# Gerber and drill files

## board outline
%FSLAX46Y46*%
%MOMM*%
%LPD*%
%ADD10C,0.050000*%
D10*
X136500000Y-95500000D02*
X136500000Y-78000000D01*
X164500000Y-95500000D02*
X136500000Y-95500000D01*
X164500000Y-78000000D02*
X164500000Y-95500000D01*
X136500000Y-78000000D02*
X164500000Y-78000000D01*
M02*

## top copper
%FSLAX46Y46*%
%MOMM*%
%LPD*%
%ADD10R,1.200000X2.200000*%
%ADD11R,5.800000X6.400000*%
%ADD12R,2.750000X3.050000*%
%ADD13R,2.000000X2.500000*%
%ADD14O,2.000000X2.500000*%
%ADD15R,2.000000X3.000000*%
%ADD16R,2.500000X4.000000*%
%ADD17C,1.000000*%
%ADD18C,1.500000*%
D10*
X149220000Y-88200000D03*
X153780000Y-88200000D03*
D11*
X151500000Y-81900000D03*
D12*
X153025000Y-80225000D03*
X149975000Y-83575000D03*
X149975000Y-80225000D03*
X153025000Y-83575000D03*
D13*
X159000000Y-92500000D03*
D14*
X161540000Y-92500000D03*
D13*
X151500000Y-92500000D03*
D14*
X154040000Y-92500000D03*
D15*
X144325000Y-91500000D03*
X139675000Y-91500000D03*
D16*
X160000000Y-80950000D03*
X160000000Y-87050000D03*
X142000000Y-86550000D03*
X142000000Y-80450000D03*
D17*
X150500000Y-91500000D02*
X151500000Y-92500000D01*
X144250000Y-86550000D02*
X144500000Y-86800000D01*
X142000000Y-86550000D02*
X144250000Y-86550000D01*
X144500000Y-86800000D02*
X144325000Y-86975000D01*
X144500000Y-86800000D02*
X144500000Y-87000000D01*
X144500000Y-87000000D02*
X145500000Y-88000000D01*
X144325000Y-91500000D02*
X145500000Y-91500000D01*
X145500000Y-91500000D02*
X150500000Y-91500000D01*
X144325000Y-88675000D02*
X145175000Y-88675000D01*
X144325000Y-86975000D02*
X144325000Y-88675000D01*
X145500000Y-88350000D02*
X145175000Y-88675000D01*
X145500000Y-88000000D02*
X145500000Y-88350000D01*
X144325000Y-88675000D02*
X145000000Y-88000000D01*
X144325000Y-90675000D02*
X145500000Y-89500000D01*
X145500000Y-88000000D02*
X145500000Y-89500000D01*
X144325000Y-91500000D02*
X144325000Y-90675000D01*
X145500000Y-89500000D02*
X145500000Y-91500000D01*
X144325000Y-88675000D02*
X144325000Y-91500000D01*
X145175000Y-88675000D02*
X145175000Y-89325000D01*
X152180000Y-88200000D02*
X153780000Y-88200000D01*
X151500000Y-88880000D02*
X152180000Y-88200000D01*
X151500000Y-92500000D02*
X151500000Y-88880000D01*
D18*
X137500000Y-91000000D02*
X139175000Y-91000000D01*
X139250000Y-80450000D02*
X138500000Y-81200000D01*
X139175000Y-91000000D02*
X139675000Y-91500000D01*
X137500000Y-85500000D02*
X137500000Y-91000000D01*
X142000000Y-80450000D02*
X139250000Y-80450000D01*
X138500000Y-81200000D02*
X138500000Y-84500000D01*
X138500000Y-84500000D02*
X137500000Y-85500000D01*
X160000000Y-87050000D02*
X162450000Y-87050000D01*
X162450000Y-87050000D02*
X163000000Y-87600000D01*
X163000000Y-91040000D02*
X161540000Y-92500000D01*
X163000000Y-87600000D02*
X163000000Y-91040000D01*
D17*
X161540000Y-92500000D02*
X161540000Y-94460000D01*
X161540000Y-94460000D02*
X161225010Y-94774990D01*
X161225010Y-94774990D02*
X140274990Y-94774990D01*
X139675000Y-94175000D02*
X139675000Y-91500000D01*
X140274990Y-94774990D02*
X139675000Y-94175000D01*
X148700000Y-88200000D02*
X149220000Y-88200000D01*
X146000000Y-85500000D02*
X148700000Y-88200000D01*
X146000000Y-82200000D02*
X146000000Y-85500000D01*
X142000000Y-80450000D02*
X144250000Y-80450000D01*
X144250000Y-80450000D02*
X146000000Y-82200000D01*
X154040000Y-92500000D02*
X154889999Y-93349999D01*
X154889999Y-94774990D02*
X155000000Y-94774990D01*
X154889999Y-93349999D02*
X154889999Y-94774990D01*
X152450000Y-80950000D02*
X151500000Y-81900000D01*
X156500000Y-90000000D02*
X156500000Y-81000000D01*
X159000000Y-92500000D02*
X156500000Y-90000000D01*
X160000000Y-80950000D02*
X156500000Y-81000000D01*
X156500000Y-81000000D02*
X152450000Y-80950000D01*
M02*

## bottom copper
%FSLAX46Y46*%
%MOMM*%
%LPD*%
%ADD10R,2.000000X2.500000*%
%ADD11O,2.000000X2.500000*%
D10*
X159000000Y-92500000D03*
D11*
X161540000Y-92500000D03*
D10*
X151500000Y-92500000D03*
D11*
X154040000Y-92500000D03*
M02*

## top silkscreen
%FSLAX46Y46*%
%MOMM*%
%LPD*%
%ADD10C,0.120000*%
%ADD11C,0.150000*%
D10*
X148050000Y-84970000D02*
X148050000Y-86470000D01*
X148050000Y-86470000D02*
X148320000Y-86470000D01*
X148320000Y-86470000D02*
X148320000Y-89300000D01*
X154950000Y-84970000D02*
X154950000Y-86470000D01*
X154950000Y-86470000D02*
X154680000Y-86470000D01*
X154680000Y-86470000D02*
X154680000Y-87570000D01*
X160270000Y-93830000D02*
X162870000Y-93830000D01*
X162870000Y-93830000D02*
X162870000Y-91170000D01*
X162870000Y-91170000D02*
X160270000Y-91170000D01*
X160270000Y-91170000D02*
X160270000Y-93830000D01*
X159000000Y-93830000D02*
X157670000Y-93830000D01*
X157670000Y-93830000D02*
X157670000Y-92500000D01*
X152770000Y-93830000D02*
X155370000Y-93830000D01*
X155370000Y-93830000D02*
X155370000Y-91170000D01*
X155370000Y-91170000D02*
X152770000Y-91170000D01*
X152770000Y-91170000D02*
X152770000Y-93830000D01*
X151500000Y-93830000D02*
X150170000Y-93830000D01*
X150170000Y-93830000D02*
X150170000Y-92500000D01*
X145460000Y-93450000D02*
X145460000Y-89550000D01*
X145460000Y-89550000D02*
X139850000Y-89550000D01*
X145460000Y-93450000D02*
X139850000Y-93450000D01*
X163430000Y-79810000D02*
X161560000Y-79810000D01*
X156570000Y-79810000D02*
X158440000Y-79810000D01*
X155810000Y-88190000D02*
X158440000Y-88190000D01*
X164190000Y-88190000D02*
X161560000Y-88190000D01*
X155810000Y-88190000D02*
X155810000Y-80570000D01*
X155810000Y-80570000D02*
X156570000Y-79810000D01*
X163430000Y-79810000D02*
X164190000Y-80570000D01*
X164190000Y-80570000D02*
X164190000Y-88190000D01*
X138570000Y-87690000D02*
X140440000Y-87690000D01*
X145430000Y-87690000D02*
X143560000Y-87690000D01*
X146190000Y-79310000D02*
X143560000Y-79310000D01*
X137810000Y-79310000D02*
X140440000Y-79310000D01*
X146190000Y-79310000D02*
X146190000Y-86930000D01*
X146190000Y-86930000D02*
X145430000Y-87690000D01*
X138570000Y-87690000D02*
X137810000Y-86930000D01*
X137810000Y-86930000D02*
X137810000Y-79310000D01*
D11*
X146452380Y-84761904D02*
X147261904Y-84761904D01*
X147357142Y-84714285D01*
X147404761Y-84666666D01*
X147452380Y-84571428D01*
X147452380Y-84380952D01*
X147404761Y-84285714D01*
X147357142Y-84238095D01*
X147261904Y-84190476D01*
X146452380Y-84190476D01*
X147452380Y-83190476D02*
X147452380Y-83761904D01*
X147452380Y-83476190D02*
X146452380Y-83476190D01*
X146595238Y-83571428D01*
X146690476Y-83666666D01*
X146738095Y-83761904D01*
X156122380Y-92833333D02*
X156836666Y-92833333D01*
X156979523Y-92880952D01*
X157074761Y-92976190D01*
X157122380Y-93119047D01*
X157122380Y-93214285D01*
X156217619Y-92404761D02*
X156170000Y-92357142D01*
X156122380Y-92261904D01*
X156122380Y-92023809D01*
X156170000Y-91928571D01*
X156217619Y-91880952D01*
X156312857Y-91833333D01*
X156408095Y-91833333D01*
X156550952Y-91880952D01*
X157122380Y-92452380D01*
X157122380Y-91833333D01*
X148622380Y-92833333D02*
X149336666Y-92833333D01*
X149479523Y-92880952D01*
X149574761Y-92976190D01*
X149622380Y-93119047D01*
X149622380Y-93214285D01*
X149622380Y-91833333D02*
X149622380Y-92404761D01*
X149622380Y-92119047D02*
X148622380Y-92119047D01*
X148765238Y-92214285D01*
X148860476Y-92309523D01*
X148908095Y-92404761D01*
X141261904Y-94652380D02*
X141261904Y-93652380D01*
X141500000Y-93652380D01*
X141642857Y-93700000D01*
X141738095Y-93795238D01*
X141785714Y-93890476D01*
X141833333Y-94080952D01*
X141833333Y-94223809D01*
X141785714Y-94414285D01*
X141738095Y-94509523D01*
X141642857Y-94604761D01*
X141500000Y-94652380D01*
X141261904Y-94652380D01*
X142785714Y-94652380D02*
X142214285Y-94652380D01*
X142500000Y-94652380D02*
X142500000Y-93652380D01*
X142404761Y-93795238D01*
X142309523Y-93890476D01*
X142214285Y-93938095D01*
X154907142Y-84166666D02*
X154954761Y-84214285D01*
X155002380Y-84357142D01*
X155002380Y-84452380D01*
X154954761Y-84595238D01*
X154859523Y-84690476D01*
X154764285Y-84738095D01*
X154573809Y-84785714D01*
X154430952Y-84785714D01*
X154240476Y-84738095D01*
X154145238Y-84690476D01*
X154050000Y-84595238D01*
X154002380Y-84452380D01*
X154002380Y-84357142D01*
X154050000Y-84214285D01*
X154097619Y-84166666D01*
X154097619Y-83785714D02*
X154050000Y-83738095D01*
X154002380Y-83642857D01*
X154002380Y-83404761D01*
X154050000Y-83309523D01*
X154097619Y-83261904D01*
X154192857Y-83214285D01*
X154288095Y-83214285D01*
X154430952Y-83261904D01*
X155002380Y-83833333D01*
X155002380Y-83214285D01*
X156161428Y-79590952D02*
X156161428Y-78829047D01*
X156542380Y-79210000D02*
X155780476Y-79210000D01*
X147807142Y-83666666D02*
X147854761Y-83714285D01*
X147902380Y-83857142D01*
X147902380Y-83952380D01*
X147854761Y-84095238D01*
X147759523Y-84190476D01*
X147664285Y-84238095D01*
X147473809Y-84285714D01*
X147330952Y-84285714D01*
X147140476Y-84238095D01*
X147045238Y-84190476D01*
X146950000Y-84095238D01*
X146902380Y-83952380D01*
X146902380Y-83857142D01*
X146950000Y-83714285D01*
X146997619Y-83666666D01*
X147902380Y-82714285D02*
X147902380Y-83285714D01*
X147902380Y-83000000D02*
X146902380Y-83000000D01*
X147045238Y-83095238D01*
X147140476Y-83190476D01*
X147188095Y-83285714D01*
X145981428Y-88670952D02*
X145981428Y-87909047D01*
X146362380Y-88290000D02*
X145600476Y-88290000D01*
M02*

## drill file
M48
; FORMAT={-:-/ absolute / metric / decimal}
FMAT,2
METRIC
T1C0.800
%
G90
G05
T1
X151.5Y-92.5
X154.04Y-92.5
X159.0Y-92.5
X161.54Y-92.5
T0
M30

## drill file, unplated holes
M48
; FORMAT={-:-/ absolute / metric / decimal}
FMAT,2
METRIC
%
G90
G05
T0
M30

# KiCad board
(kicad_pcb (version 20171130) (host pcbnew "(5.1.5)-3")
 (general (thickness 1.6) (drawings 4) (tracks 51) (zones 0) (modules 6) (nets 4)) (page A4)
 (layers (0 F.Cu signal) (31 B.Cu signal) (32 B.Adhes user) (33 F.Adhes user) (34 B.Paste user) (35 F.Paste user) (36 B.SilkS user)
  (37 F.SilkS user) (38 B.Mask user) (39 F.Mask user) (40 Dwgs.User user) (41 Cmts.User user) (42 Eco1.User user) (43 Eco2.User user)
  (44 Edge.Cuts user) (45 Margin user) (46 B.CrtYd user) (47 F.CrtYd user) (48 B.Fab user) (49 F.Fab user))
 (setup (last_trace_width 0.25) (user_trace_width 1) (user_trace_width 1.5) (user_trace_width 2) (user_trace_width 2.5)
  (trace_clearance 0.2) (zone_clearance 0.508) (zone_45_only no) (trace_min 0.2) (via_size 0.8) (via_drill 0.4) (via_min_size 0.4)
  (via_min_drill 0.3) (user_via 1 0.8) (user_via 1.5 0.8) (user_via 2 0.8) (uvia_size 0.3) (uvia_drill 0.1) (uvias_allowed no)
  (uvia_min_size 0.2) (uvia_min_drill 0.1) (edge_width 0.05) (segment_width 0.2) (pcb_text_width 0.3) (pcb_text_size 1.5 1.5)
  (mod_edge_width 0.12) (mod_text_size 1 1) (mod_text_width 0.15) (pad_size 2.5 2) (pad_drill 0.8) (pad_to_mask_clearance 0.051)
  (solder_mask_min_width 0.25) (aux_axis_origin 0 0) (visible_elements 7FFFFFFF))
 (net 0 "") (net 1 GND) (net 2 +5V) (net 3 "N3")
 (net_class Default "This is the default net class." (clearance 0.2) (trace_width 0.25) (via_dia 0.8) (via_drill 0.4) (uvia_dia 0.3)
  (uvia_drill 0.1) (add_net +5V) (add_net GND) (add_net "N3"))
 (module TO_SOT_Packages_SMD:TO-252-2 (layer F.Cu) (at 151.5 84 90)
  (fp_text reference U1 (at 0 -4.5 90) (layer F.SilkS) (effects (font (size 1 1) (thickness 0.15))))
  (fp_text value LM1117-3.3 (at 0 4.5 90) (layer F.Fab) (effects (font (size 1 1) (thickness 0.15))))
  (fp_line (start -0.97 -3.45) (end -2.47 -3.45) (layer F.SilkS) (width 0.12))
  (fp_line (start -2.47 -3.45) (end -2.47 -3.18) (layer F.SilkS) (width 0.12))
  (fp_line (start -2.47 -3.18) (end -5.3 -3.18) (layer F.SilkS) (width 0.12))
  (fp_line (start -0.97 3.45) (end -2.47 3.45) (layer F.SilkS) (width 0.12))
  (fp_line (start -2.47 3.45) (end -2.47 3.18) (layer F.SilkS) (width 0.12))
  (fp_line (start -2.47 3.18) (end -3.57 3.18) (layer F.SilkS) (width 0.12))
  (pad 1 smd rect (at -4.2 -2.28 90) (size 2.2 1.2) (layers F.Cu F.Paste F.Mask) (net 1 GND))
  (pad 3 smd rect (at -4.2 2.28 90) (size 2.2 1.2) (layers F.Cu F.Paste F.Mask) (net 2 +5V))
  (pad 2 smd rect (at 2.1 0 90) (size 6.4 5.8) (layers F.Cu F.Mask) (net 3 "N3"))
  (pad 2 smd rect (at 3.775 1.525 90) (size 3.05 2.75) (layers F.Cu F.Paste) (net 3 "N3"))
  (pad 2 smd rect (at 0.425 -1.525 90) (size 3.05 2.75) (layers F.Cu F.Paste) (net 3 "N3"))
  (pad 2 smd rect (at 3.775 -1.525 90) (size 3.05 2.75) (layers F.Cu F.Paste) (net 3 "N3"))
  (pad 2 smd rect (at 0.425 1.525 90) (size 3.05 2.75) (layers F.Cu F.Paste) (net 3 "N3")))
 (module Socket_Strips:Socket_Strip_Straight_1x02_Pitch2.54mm (layer F.Cu) (at 159 92.5 90)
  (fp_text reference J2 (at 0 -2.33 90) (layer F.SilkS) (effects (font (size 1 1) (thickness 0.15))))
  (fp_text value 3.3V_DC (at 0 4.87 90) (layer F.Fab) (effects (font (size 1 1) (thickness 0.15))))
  (fp_line (start -1.33 1.27) (end -1.33 3.87) (layer F.SilkS) (width 0.12))
  (fp_line (start -1.33 3.87) (end 1.33 3.87) (layer F.SilkS) (width 0.12))
  (fp_line (start 1.33 3.87) (end 1.33 1.27) (layer F.SilkS) (width 0.12))
  (fp_line (start 1.33 1.27) (end -1.33 1.27) (layer F.SilkS) (width 0.12))
  (fp_line (start -1.33 0) (end -1.33 -1.33) (layer F.SilkS) (width 0.12))
  (fp_line (start -1.33 -1.33) (end 0 -1.33) (layer F.SilkS) (width 0.12))
  (pad 1 thru_hole rect (at 0 0 90) (size 2.5 2) (drill 0.8) (layers *.Cu *.Mask) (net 3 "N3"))
  (pad 2 thru_hole oval (at 0 2.54 90) (size 2.5 2) (drill 0.8) (layers *.Cu *.Mask) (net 1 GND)))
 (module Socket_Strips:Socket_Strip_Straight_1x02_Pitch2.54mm (layer F.Cu) (at 151.5 92.5 90)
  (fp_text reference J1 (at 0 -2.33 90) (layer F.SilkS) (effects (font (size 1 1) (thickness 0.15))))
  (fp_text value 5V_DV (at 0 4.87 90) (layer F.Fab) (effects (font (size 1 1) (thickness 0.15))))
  (fp_line (start -1.33 1.27) (end -1.33 3.87) (layer F.SilkS) (width 0.12))
  (fp_line (start -1.33 3.87) (end 1.33 3.87) (layer F.SilkS) (width 0.12))
  (fp_line (start 1.33 3.87) (end 1.33 1.27) (layer F.SilkS) (width 0.12))
  (fp_line (start 1.33 1.27) (end -1.33 1.27) (layer F.SilkS) (width 0.12))
  (fp_line (start -1.33 0) (end -1.33 -1.33) (layer F.SilkS) (width 0.12))
  (fp_line (start -1.33 -1.33) (end 0 -1.33) (layer F.SilkS) (width 0.12))
  (pad 1 thru_hole rect (at 0 0 90) (size 2.5 2) (drill 0.8) (layers *.Cu *.Mask) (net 2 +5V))
  (pad 2 thru_hole oval (at 0 2.54 90) (size 2.5 2) (drill 0.8) (layers *.Cu *.Mask) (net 1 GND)))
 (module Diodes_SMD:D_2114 (layer F.Cu) (at 142 91.5 180)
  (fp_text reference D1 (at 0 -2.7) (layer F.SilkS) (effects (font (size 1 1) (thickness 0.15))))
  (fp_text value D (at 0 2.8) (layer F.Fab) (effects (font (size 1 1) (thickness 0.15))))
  (fp_line (start -3.46 -1.95) (end -3.46 1.95) (layer F.SilkS) (width 0.12))
  (fp_line (start -3.46 1.95) (end 2.15 1.95) (layer F.SilkS) (width 0.12))
  (fp_line (start -3.46 -1.95) (end 2.15 -1.95) (layer F.SilkS) (width 0.12))
  (pad 1 smd rect (at -2.325 0 180) (size 2 3) (layers F.Cu F.Paste F.Mask) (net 2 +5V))
  (pad 2 smd rect (at 2.325 0 180) (size 2 3) (layers F.Cu F.Paste F.Mask) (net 1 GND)))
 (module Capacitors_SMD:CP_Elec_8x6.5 (layer F.Cu) (at 160 84 270)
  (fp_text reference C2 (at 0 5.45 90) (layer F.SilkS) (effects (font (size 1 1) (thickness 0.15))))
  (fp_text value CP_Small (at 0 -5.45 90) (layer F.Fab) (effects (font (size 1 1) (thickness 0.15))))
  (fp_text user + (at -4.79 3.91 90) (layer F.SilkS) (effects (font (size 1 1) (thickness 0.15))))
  (fp_line (start -4.19 -3.43) (end -4.19 -1.56) (layer F.SilkS) (width 0.12))
  (fp_line (start -4.19 3.43) (end -4.19 1.56) (layer F.SilkS) (width 0.12))
  (fp_line (start 4.19 4.19) (end 4.19 1.56) (layer F.SilkS) (width 0.12))
  (fp_line (start 4.19 -4.19) (end 4.19 -1.56) (layer F.SilkS) (width 0.12))
  (fp_line (start 4.19 4.19) (end -3.43 4.19) (layer F.SilkS) (width 0.12))
  (fp_line (start -3.43 4.19) (end -4.19 3.43) (layer F.SilkS) (width 0.12))
  (fp_line (start -4.19 -3.43) (end -3.43 -4.19) (layer F.SilkS) (width 0.12))
  (fp_line (start -3.43 -4.19) (end 4.19 -4.19) (layer F.SilkS) (width 0.12))
  (pad 1 smd rect (at -3.05 0 90) (size 4 2.5) (layers F.Cu F.Paste F.Mask) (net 3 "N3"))
  (pad 2 smd rect (at 3.05 0 90) (size 4 2.5) (layers F.Cu F.Paste F.Mask) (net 1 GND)))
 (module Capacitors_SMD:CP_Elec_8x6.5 (layer F.Cu) (at 142 83.5 90)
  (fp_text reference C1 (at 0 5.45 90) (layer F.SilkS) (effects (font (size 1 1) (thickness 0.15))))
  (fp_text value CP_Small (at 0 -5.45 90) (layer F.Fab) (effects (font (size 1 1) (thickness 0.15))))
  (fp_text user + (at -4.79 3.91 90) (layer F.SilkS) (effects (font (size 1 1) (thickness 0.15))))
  (fp_line (start -4.19 -3.43) (end -4.19 -1.56) (layer F.SilkS) (width 0.12))
  (fp_line (start -4.19 3.43) (end -4.19 1.56) (layer F.SilkS) (width 0.12))
  (fp_line (start 4.19 4.19) (end 4.19 1.56) (layer F.SilkS) (width 0.12))
  (fp_line (start 4.19 -4.19) (end 4.19 -1.56) (layer F.SilkS) (width 0.12))
  (fp_line (start 4.19 4.19) (end -3.43 4.19) (layer F.SilkS) (width 0.12))
  (fp_line (start -3.43 4.19) (end -4.19 3.43) (layer F.SilkS) (width 0.12))
  (fp_line (start -4.19 -3.43) (end -3.43 -4.19) (layer F.SilkS) (width 0.12))
  (fp_line (start -3.43 -4.19) (end 4.19 -4.19) (layer F.SilkS) (width 0.12))
  (pad 1 smd rect (at -3.05 0 270) (size 4 2.5) (layers F.Cu F.Paste F.Mask) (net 2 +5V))
  (pad 2 smd rect (at 3.05 0 270) (size 4 2.5) (layers F.Cu F.Paste F.Mask) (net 1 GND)))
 (gr_line (start 136.5 95.5) (end 136.5 78) (layer Edge.Cuts) (width 0.05))
 (gr_line (start 164.5 95.5) (end 136.5 95.5) (layer Edge.Cuts) (width 0.05))
 (gr_line (start 164.5 78) (end 164.5 95.5) (layer Edge.Cuts) (width 0.05))
 (gr_line (start 136.5 78) (end 164.5 78) (layer Edge.Cuts) (width 0.05))
 (segment (start 150.5 91.5) (end 151.5 92.5) (width 1) (layer F.Cu) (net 2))
 (segment (start 144.25 86.55) (end 144.5 86.8) (width 1) (layer F.Cu) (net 2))
 (segment (start 142 86.55) (end 144.25 86.55) (width 1) (layer F.Cu) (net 2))
 (segment (start 144.5 86.8) (end 144.325 86.975) (width 1) (layer F.Cu) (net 2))
 (segment (start 144.5 86.8) (end 144.5 87) (width 1) (layer F.Cu) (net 2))
 (segment (start 144.5 87) (end 145.5 88) (width 1) (layer F.Cu) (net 2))
 (segment (start 144.325 91.5) (end 145.5 91.5) (width 1) (layer F.Cu) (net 2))
 (segment (start 145.5 91.5) (end 150.5 91.5) (width 1) (layer F.Cu) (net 2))
 (segment (start 144.325 88.675) (end 145.175 88.675) (width 1) (layer F.Cu) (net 2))
 (segment (start 144.325 86.975) (end 144.325 88.675) (width 1) (layer F.Cu) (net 2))
 (segment (start 145.5 88.35) (end 145.175 88.675) (width 1) (layer F.Cu) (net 2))
 (segment (start 145.5 88) (end 145.5 88.35) (width 1) (layer F.Cu) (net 2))
 (segment (start 144.325 88.675) (end 145 88) (width 1) (layer F.Cu) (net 2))
 (segment (start 144.325 90.675) (end 145.5 89.5) (width 1) (layer F.Cu) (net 2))
 (segment (start 145.5 88) (end 145.5 89.5) (width 1) (layer F.Cu) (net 2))
 (segment (start 144.325 91.5) (end 144.325 90.675) (width 1) (layer F.Cu) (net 2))
 (segment (start 145.5 89.5) (end 145.5 91.5) (width 1) (layer F.Cu) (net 2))
 (segment (start 144.325 88.675) (end 144.325 91.5) (width 1) (layer F.Cu) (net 2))
 (segment (start 145.175 88.675) (end 145.175 89.325) (width 1) (layer F.Cu) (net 2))
 (segment (start 152.18 88.2) (end 153.78 88.2) (width 1) (layer F.Cu) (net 2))
 (segment (start 151.5 88.88) (end 152.18 88.2) (width 1) (layer F.Cu) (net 2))
 (segment (start 151.5 92.5) (end 151.5 88.88) (width 1) (layer F.Cu) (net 2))
 (segment (start 137.5 91) (end 139.175 91) (width 1.5) (layer F.Cu) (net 1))
 (segment (start 139.25 80.45) (end 138.5 81.2) (width 1.5) (layer F.Cu) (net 1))
 (segment (start 139.175 91) (end 139.675 91.5) (width 1.5) (layer F.Cu) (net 1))
 (segment (start 137.5 85.5) (end 137.5 91) (width 1.5) (layer F.Cu) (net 1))
 (segment (start 142 80.45) (end 139.25 80.45) (width 1.5) (layer F.Cu) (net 1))
 (segment (start 138.5 81.2) (end 138.5 84.5) (width 1.5) (layer F.Cu) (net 1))
 (segment (start 138.5 84.5) (end 137.5 85.5) (width 1.5) (layer F.Cu) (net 1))
 (segment (start 160 87.05) (end 162.45 87.05) (width 1.5) (layer F.Cu) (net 1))
 (segment (start 162.45 87.05) (end 163 87.6) (width 1.5) (layer F.Cu) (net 1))
 (segment (start 163 91.04) (end 161.54 92.5) (width 1.5) (layer F.Cu) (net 1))
 (segment (start 163 87.6) (end 163 91.04) (width 1.5) (layer F.Cu) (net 1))
 (segment (start 161.54 92.5) (end 161.54 94.46) (width 1) (layer F.Cu) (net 1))
 (segment (start 161.54 94.46) (end 161.22501 94.77499) (width 1) (layer F.Cu) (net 1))
 (segment (start 161.22501 94.77499) (end 140.27499 94.77499) (width 1) (layer F.Cu) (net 1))
 (segment (start 139.675 94.175) (end 139.675 91.5) (width 1) (layer F.Cu) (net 1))
 (segment (start 140.27499 94.77499) (end 139.675 94.175) (width 1) (layer F.Cu) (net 1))
 (segment (start 148.7 88.2) (end 149.22 88.2) (width 1) (layer F.Cu) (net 1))
 (segment (start 146 85.5) (end 148.7 88.2) (width 1) (layer F.Cu) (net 1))
 (segment (start 146 82.2) (end 146 85.5) (width 1) (layer F.Cu) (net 1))
 (segment (start 142 80.45) (end 144.25 80.45) (width 1) (layer F.Cu) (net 1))
 (segment (start 144.25 80.45) (end 146 82.2) (width 1) (layer F.Cu) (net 1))
 (segment (start 154.04 92.5) (end 154.889999 93.349999) (width 1) (layer F.Cu) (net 1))
 (segment (start 154.889999 94.77499) (end 155 94.77499) (width 1) (layer F.Cu) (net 1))
 (segment (start 154.889999 93.349999) (end 154.889999 94.77499) (width 1) (layer F.Cu) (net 1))
 (segment (start 152.45 80.95) (end 151.5 81.9) (width 1) (layer F.Cu) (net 3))
 (segment (start 156.5 90) (end 156.5 81) (width 1) (layer F.Cu) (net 3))
 (segment (start 159 92.5) (end 156.5 90) (width 1) (layer F.Cu) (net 3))
 (segment (start 160 80.95) (end 156.5 81) (width 1) (layer F.Cu) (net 3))
 (segment (start 156.5 81) (end 152.45 80.95) (width 1) (layer F.Cu) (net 3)))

